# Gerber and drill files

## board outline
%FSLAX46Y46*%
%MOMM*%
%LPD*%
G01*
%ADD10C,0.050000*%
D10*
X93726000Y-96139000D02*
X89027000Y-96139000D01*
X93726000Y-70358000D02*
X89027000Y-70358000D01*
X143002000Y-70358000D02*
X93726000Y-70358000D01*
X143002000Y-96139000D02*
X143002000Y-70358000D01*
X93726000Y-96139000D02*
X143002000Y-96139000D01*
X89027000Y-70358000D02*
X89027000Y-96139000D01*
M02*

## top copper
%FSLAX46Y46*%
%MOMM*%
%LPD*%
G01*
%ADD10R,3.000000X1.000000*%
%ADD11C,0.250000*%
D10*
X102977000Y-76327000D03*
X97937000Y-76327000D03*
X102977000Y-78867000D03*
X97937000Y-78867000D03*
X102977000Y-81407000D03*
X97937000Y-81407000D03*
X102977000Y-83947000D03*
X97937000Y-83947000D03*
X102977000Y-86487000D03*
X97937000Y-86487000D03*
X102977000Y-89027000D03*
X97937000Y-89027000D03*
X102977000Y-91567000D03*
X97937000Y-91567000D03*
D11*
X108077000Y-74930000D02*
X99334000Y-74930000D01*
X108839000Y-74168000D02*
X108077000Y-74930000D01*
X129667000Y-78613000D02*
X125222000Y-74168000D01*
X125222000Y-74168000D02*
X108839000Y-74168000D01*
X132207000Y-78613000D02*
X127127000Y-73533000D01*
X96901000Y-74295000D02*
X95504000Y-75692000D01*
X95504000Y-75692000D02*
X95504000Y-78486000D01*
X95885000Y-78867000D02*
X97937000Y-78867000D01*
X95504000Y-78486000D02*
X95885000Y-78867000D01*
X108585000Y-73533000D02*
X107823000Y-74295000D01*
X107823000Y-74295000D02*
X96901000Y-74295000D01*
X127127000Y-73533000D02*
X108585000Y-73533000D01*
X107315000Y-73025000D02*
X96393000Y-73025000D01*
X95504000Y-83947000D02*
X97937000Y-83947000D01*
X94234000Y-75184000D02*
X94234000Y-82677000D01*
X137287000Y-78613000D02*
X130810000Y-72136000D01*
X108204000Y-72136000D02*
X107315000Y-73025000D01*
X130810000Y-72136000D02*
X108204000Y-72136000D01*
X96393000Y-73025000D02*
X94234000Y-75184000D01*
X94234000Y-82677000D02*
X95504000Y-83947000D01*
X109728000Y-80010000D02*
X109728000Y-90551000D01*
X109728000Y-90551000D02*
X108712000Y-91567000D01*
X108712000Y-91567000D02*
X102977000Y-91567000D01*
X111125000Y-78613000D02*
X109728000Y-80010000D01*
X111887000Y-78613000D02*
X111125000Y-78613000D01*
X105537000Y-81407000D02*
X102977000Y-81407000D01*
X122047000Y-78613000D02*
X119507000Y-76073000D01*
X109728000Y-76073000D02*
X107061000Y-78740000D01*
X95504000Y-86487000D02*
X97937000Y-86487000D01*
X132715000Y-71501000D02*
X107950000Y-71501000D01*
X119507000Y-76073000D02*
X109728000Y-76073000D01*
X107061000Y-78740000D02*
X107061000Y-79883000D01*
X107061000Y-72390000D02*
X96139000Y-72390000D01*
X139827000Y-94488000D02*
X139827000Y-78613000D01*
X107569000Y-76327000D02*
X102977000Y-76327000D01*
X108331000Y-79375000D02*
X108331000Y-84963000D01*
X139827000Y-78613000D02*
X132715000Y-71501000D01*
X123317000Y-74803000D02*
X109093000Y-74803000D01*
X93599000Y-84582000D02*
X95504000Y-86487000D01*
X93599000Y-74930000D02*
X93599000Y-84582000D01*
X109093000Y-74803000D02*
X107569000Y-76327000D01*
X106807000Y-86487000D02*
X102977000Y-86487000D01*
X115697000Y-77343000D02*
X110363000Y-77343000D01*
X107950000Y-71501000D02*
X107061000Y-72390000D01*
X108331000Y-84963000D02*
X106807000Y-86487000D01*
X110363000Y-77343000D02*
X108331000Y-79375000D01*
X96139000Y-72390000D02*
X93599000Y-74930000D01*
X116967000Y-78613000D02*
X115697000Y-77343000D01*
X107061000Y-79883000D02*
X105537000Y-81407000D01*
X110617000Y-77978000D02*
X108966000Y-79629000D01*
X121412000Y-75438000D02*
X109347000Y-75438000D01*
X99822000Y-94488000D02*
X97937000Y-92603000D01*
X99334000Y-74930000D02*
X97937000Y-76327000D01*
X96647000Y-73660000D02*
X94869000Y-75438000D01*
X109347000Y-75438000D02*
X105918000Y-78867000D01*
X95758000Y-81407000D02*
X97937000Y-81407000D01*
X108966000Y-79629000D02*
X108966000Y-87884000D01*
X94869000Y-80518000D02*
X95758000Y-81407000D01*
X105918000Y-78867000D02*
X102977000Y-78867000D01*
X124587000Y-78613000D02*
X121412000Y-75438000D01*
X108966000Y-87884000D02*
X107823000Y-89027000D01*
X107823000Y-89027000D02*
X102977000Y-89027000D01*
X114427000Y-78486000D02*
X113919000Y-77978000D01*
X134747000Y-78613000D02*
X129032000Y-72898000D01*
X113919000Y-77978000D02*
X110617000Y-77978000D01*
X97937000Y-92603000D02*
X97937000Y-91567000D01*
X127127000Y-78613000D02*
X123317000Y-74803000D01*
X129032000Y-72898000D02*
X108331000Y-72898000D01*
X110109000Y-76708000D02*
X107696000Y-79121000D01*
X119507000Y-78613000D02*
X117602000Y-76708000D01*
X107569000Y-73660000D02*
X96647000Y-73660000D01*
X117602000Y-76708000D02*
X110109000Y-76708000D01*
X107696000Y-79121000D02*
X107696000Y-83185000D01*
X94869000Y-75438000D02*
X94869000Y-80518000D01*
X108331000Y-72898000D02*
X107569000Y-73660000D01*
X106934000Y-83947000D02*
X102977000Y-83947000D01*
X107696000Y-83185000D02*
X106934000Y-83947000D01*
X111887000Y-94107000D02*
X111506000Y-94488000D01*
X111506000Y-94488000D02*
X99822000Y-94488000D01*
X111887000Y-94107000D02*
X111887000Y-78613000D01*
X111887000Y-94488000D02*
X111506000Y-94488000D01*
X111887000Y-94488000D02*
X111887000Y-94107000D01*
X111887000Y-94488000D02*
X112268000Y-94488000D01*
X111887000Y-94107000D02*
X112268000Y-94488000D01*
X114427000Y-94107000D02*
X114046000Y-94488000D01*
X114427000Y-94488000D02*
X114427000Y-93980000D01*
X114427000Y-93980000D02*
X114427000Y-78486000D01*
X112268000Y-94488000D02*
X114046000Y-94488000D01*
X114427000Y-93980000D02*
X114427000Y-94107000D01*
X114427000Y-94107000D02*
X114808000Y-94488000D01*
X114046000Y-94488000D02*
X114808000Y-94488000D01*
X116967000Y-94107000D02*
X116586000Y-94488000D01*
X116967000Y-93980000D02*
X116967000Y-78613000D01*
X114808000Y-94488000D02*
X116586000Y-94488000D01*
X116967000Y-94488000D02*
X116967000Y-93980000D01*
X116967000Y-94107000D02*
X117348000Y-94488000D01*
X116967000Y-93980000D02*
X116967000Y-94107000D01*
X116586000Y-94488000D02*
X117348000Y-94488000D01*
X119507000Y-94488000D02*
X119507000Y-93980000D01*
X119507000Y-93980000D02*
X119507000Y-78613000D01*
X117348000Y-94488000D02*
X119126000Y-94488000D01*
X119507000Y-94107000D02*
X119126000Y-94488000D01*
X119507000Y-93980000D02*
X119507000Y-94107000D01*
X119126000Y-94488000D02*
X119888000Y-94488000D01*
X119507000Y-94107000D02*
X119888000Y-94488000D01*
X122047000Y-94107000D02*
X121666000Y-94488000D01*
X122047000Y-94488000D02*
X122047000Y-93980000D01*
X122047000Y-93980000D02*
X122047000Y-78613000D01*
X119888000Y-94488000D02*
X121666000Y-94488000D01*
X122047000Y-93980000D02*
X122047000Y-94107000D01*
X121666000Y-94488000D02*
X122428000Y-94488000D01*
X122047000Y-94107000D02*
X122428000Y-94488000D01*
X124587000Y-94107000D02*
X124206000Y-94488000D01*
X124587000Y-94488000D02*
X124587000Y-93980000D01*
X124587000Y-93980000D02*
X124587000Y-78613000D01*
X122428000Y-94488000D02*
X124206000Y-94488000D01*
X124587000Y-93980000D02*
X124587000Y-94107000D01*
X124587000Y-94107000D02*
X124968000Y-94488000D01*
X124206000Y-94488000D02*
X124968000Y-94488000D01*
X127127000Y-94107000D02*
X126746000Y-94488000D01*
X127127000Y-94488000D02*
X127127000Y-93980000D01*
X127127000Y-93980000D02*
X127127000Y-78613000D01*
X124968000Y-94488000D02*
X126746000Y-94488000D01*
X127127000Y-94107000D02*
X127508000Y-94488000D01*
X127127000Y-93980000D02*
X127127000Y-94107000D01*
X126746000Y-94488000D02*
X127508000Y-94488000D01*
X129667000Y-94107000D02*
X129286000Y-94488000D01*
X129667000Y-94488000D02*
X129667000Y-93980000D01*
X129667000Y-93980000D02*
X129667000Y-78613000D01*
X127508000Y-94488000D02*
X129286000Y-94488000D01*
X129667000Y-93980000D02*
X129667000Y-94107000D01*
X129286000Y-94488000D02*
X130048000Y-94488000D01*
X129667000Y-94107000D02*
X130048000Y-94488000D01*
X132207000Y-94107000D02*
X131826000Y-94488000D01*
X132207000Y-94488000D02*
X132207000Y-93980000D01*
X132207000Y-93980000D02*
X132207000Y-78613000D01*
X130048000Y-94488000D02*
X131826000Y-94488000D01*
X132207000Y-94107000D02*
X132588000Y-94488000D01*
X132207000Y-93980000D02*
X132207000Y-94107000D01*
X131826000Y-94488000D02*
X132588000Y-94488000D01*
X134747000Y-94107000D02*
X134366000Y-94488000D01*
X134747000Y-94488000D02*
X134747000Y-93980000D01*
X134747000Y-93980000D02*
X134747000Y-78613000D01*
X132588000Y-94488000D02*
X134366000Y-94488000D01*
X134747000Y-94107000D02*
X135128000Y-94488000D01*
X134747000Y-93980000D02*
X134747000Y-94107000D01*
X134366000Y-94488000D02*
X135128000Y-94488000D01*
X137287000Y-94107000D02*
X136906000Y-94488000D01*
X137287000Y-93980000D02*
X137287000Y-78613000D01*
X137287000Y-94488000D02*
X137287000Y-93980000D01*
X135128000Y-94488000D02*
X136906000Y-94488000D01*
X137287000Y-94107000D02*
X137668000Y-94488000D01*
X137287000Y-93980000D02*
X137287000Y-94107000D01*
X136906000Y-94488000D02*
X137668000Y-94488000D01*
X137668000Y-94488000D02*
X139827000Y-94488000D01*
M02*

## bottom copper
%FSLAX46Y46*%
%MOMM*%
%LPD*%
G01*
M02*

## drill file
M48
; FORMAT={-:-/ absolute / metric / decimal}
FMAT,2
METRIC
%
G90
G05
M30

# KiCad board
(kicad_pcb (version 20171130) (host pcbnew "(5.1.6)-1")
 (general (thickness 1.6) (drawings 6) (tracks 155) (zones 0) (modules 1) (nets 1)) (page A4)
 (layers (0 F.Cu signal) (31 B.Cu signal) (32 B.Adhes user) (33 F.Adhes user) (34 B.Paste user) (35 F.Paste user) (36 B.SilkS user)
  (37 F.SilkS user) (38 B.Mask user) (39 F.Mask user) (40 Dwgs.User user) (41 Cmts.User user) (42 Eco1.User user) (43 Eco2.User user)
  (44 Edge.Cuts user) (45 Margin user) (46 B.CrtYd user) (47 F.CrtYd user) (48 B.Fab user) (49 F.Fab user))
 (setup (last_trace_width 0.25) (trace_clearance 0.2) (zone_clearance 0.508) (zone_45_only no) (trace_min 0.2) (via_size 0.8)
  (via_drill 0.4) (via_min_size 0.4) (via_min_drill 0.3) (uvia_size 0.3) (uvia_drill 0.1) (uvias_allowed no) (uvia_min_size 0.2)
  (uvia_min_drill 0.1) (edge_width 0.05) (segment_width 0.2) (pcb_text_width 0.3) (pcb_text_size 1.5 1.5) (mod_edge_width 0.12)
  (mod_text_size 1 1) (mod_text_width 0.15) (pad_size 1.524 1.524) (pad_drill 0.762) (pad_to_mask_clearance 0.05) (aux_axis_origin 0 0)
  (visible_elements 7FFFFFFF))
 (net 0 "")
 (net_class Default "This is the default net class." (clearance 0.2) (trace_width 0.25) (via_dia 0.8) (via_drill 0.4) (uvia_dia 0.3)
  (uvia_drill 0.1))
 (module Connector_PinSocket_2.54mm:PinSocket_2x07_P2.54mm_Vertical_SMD (layer F.Cu) (at 100.457 83.947)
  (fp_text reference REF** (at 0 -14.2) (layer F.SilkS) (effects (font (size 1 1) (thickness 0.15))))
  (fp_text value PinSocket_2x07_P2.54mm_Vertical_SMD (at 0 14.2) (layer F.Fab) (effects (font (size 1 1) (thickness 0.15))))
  (pad 1 smd rect (at 2.52 -7.62) (size 3 1) (layers F.Cu F.Paste F.Mask))
  (pad 2 smd rect (at -2.52 -7.62) (size 3 1) (layers F.Cu F.Paste F.Mask))
  (pad 3 smd rect (at 2.52 -5.08) (size 3 1) (layers F.Cu F.Paste F.Mask))
  (pad 4 smd rect (at -2.52 -5.08) (size 3 1) (layers F.Cu F.Paste F.Mask))
  (pad 5 smd rect (at 2.52 -2.54) (size 3 1) (layers F.Cu F.Paste F.Mask))
  (pad 6 smd rect (at -2.52 -2.54) (size 3 1) (layers F.Cu F.Paste F.Mask))
  (pad 7 smd rect (at 2.52 0) (size 3 1) (layers F.Cu F.Paste F.Mask))
  (pad 8 smd rect (at -2.52 0) (size 3 1) (layers F.Cu F.Paste F.Mask))
  (pad 9 smd rect (at 2.52 2.54) (size 3 1) (layers F.Cu F.Paste F.Mask))
  (pad 10 smd rect (at -2.52 2.54) (size 3 1) (layers F.Cu F.Paste F.Mask))
  (pad 11 smd rect (at 2.52 5.08) (size 3 1) (layers F.Cu F.Paste F.Mask))
  (pad 12 smd rect (at -2.52 5.08) (size 3 1) (layers F.Cu F.Paste F.Mask))
  (pad 13 smd rect (at 2.52 7.62) (size 3 1) (layers F.Cu F.Paste F.Mask))
  (pad 14 smd rect (at -2.52 7.62) (size 3 1) (layers F.Cu F.Paste F.Mask)))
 (gr_line (start 93.726 96.139) (end 89.027 96.139) (layer Edge.Cuts) (width 0.05))
 (gr_line (start 93.726 70.358) (end 89.027 70.358) (layer Edge.Cuts) (width 0.05))
 (gr_line (start 143.002 70.358) (end 93.726 70.358) (layer Edge.Cuts) (width 0.05))
 (gr_line (start 143.002 96.139) (end 143.002 70.358) (layer Edge.Cuts) (width 0.05))
 (gr_line (start 93.726 96.139) (end 143.002 96.139) (layer Edge.Cuts) (width 0.05))
 (gr_line (start 89.027 70.358) (end 89.027 96.139) (layer Edge.Cuts) (width 0.05))
 (segment (start 108.077 74.93) (end 99.334 74.93) (width 0.25) (layer F.Cu) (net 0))
 (segment (start 108.839 74.168) (end 108.077 74.93) (width 0.25) (layer F.Cu) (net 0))
 (segment (start 129.667 78.613) (end 125.222 74.168) (width 0.25) (layer F.Cu) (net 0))
 (segment (start 125.222 74.168) (end 108.839 74.168) (width 0.25) (layer F.Cu) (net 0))
 (segment (start 132.207 78.613) (end 127.127 73.533) (width 0.25) (layer F.Cu) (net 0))
 (segment (start 96.901 74.295) (end 95.504 75.692) (width 0.25) (layer F.Cu) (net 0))
 (segment (start 95.504 75.692) (end 95.504 78.486) (width 0.25) (layer F.Cu) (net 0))
 (segment (start 95.885 78.867) (end 97.937 78.867) (width 0.25) (layer F.Cu) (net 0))
 (segment (start 95.504 78.486) (end 95.885 78.867) (width 0.25) (layer F.Cu) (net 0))
 (segment (start 108.585 73.533) (end 107.823 74.295) (width 0.25) (layer F.Cu) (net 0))
 (segment (start 107.823 74.295) (end 96.901 74.295) (width 0.25) (layer F.Cu) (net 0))
 (segment (start 127.127 73.533) (end 108.585 73.533) (width 0.25) (layer F.Cu) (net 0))
 (segment (start 107.315 73.025) (end 96.393 73.025) (width 0.25) (layer F.Cu) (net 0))
 (segment (start 95.504 83.947) (end 97.937 83.947) (width 0.25) (layer F.Cu) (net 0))
 (segment (start 94.234 75.184) (end 94.234 82.677) (width 0.25) (layer F.Cu) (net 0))
 (segment (start 137.287 78.613) (end 130.81 72.136) (width 0.25) (layer F.Cu) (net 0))
 (segment (start 108.204 72.136) (end 107.315 73.025) (width 0.25) (layer F.Cu) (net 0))
 (segment (start 130.81 72.136) (end 108.204 72.136) (width 0.25) (layer F.Cu) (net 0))
 (segment (start 96.393 73.025) (end 94.234 75.184) (width 0.25) (layer F.Cu) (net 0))
 (segment (start 94.234 82.677) (end 95.504 83.947) (width 0.25) (layer F.Cu) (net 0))
 (segment (start 109.728 80.01) (end 109.728 90.551) (width 0.25) (layer F.Cu) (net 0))
 (segment (start 109.728 90.551) (end 108.712 91.567) (width 0.25) (layer F.Cu) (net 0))
 (segment (start 108.712 91.567) (end 102.977 91.567) (width 0.25) (layer F.Cu) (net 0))
 (segment (start 111.125 78.613) (end 109.728 80.01) (width 0.25) (layer F.Cu) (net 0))
 (segment (start 111.887 78.613) (end 111.125 78.613) (width 0.25) (layer F.Cu) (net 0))
 (segment (start 105.537 81.407) (end 102.977 81.407) (width 0.25) (layer F.Cu) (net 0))
 (segment (start 122.047 78.613) (end 119.507 76.073) (width 0.25) (layer F.Cu) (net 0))
 (segment (start 109.728 76.073) (end 107.061 78.74) (width 0.25) (layer F.Cu) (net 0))
 (segment (start 95.504 86.487) (end 97.937 86.487) (width 0.25) (layer F.Cu) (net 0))
 (segment (start 132.715 71.501) (end 107.95 71.501) (width 0.25) (layer F.Cu) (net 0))
 (segment (start 119.507 76.073) (end 109.728 76.073) (width 0.25) (layer F.Cu) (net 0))
 (segment (start 107.061 78.74) (end 107.061 79.883) (width 0.25) (layer F.Cu) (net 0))
 (segment (start 107.061 72.39) (end 96.139 72.39) (width 0.25) (layer F.Cu) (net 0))
 (segment (start 139.827 94.488) (end 139.827 78.613) (width 0.25) (layer F.Cu) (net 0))
 (segment (start 107.569 76.327) (end 102.977 76.327) (width 0.25) (layer F.Cu) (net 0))
 (segment (start 108.331 79.375) (end 108.331 84.963) (width 0.25) (layer F.Cu) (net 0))
 (segment (start 139.827 78.613) (end 132.715 71.501) (width 0.25) (layer F.Cu) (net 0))
 (segment (start 123.317 74.803) (end 109.093 74.803) (width 0.25) (layer F.Cu) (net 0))
 (segment (start 93.599 84.582) (end 95.504 86.487) (width 0.25) (layer F.Cu) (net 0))
 (segment (start 93.599 74.93) (end 93.599 84.582) (width 0.25) (layer F.Cu) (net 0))
 (segment (start 109.093 74.803) (end 107.569 76.327) (width 0.25) (layer F.Cu) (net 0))
 (segment (start 106.807 86.487) (end 102.977 86.487) (width 0.25) (layer F.Cu) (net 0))
 (segment (start 115.697 77.343) (end 110.363 77.343) (width 0.25) (layer F.Cu) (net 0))
 (segment (start 107.95 71.501) (end 107.061 72.39) (width 0.25) (layer F.Cu) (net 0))
 (segment (start 108.331 84.963) (end 106.807 86.487) (width 0.25) (layer F.Cu) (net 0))
 (segment (start 110.363 77.343) (end 108.331 79.375) (width 0.25) (layer F.Cu) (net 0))
 (segment (start 96.139 72.39) (end 93.599 74.93) (width 0.25) (layer F.Cu) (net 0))
 (segment (start 116.967 78.613) (end 115.697 77.343) (width 0.25) (layer F.Cu) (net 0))
 (segment (start 107.061 79.883) (end 105.537 81.407) (width 0.25) (layer F.Cu) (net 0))
 (segment (start 110.617 77.978) (end 108.966 79.629) (width 0.25) (layer F.Cu) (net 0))
 (segment (start 121.412 75.438) (end 109.347 75.438) (width 0.25) (layer F.Cu) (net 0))
 (segment (start 99.822 94.488) (end 97.937 92.603) (width 0.25) (layer F.Cu) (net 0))
 (segment (start 99.334 74.93) (end 97.937 76.327) (width 0.25) (layer F.Cu) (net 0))
 (segment (start 96.647 73.66) (end 94.869 75.438) (width 0.25) (layer F.Cu) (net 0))
 (segment (start 109.347 75.438) (end 105.918 78.867) (width 0.25) (layer F.Cu) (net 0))
 (segment (start 95.758 81.407) (end 97.937 81.407) (width 0.25) (layer F.Cu) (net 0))
 (segment (start 108.966 79.629) (end 108.966 87.884) (width 0.25) (layer F.Cu) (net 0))
 (segment (start 94.869 80.518) (end 95.758 81.407) (width 0.25) (layer F.Cu) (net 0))
 (segment (start 105.918 78.867) (end 102.977 78.867) (width 0.25) (layer F.Cu) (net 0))
 (segment (start 124.587 78.613) (end 121.412 75.438) (width 0.25) (layer F.Cu) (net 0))
 (segment (start 108.966 87.884) (end 107.823 89.027) (width 0.25) (layer F.Cu) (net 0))
 (segment (start 107.823 89.027) (end 102.977 89.027) (width 0.25) (layer F.Cu) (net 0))
 (segment (start 114.427 78.486) (end 113.919 77.978) (width 0.25) (layer F.Cu) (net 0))
 (segment (start 134.747 78.613) (end 129.032 72.898) (width 0.25) (layer F.Cu) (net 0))
 (segment (start 113.919 77.978) (end 110.617 77.978) (width 0.25) (layer F.Cu) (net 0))
 (segment (start 97.937 92.603) (end 97.937 91.567) (width 0.25) (layer F.Cu) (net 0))
 (segment (start 127.127 78.613) (end 123.317 74.803) (width 0.25) (layer F.Cu) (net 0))
 (segment (start 129.032 72.898) (end 108.331 72.898) (width 0.25) (layer F.Cu) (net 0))
 (segment (start 110.109 76.708) (end 107.696 79.121) (width 0.25) (layer F.Cu) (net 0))
 (segment (start 119.507 78.613) (end 117.602 76.708) (width 0.25) (layer F.Cu) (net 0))
 (segment (start 107.569 73.66) (end 96.647 73.66) (width 0.25) (layer F.Cu) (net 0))
 (segment (start 117.602 76.708) (end 110.109 76.708) (width 0.25) (layer F.Cu) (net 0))
 (segment (start 107.696 79.121) (end 107.696 83.185) (width 0.25) (layer F.Cu) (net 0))
 (segment (start 94.869 75.438) (end 94.869 80.518) (width 0.25) (layer F.Cu) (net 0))
 (segment (start 108.331 72.898) (end 107.569 73.66) (width 0.25) (layer F.Cu) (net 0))
 (segment (start 106.934 83.947) (end 102.977 83.947) (width 0.25) (layer F.Cu) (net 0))
 (segment (start 107.696 83.185) (end 106.934 83.947) (width 0.25) (layer F.Cu) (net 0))
 (segment (start 111.887 94.107) (end 111.506 94.488) (width 0.25) (layer F.Cu) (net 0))
 (segment (start 111.506 94.488) (end 99.822 94.488) (width 0.25) (layer F.Cu) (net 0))
 (segment (start 111.887 94.107) (end 111.887 78.613) (width 0.25) (layer F.Cu) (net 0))
 (segment (start 111.887 94.488) (end 111.506 94.488) (width 0.25) (layer F.Cu) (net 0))
 (segment (start 111.887 94.488) (end 111.887 94.107) (width 0.25) (layer F.Cu) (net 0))
 (segment (start 111.887 94.488) (end 112.268 94.488) (width 0.25) (layer F.Cu) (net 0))
 (segment (start 111.887 94.107) (end 112.268 94.488) (width 0.25) (layer F.Cu) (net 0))
 (segment (start 114.427 94.107) (end 114.046 94.488) (width 0.25) (layer F.Cu) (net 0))
 (segment (start 114.427 94.488) (end 114.427 93.98) (width 0.25) (layer F.Cu) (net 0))
 (segment (start 114.427 93.98) (end 114.427 78.486) (width 0.25) (layer F.Cu) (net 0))
 (segment (start 112.268 94.488) (end 114.046 94.488) (width 0.25) (layer F.Cu) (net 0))
 (segment (start 114.427 93.98) (end 114.427 94.107) (width 0.25) (layer F.Cu) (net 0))
 (segment (start 114.427 94.107) (end 114.808 94.488) (width 0.25) (layer F.Cu) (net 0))
 (segment (start 114.046 94.488) (end 114.808 94.488) (width 0.25) (layer F.Cu) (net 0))
 (segment (start 116.967 94.107) (end 116.586 94.488) (width 0.25) (layer F.Cu) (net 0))
 (segment (start 116.967 93.98) (end 116.967 78.613) (width 0.25) (layer F.Cu) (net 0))
 (segment (start 114.808 94.488) (end 116.586 94.488) (width 0.25) (layer F.Cu) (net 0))
 (segment (start 116.967 94.488) (end 116.967 93.98) (width 0.25) (layer F.Cu) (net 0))
 (segment (start 116.967 94.107) (end 117.348 94.488) (width 0.25) (layer F.Cu) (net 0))
 (segment (start 116.967 93.98) (end 116.967 94.107) (width 0.25) (layer F.Cu) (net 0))
 (segment (start 116.586 94.488) (end 117.348 94.488) (width 0.25) (layer F.Cu) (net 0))
 (segment (start 119.507 94.488) (end 119.507 93.98) (width 0.25) (layer F.Cu) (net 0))
 (segment (start 119.507 93.98) (end 119.507 78.613) (width 0.25) (layer F.Cu) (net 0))
 (segment (start 117.348 94.488) (end 119.126 94.488) (width 0.25) (layer F.Cu) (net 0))
 (segment (start 119.507 94.107) (end 119.126 94.488) (width 0.25) (layer F.Cu) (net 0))
 (segment (start 119.507 93.98) (end 119.507 94.107) (width 0.25) (layer F.Cu) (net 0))
 (segment (start 119.126 94.488) (end 119.888 94.488) (width 0.25) (layer F.Cu) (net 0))
 (segment (start 119.507 94.107) (end 119.888 94.488) (width 0.25) (layer F.Cu) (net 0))
 (segment (start 122.047 94.107) (end 121.666 94.488) (width 0.25) (layer F.Cu) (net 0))
 (segment (start 122.047 94.488) (end 122.047 93.98) (width 0.25) (layer F.Cu) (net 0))
 (segment (start 122.047 93.98) (end 122.047 78.613) (width 0.25) (layer F.Cu) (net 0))
 (segment (start 119.888 94.488) (end 121.666 94.488) (width 0.25) (layer F.Cu) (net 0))
 (segment (start 122.047 93.98) (end 122.047 94.107) (width 0.25) (layer F.Cu) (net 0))
 (segment (start 121.666 94.488) (end 122.428 94.488) (width 0.25) (layer F.Cu) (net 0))
 (segment (start 122.047 94.107) (end 122.428 94.488) (width 0.25) (layer F.Cu) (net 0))
 (segment (start 124.587 94.107) (end 124.206 94.488) (width 0.25) (layer F.Cu) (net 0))
 (segment (start 124.587 94.488) (end 124.587 93.98) (width 0.25) (layer F.Cu) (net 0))
 (segment (start 124.587 93.98) (end 124.587 78.613) (width 0.25) (layer F.Cu) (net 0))
 (segment (start 122.428 94.488) (end 124.206 94.488) (width 0.25) (layer F.Cu) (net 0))
 (segment (start 124.587 93.98) (end 124.587 94.107) (width 0.25) (layer F.Cu) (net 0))
 (segment (start 124.587 94.107) (end 124.968 94.488) (width 0.25) (layer F.Cu) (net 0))
 (segment (start 124.206 94.488) (end 124.968 94.488) (width 0.25) (layer F.Cu) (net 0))
 (segment (start 127.127 94.107) (end 126.746 94.488) (width 0.25) (layer F.Cu) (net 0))
 (segment (start 127.127 94.488) (end 127.127 93.98) (width 0.25) (layer F.Cu) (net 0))
 (segment (start 127.127 93.98) (end 127.127 78.613) (width 0.25) (layer F.Cu) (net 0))
 (segment (start 124.968 94.488) (end 126.746 94.488) (width 0.25) (layer F.Cu) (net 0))
 (segment (start 127.127 94.107) (end 127.508 94.488) (width 0.25) (layer F.Cu) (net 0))
 (segment (start 127.127 93.98) (end 127.127 94.107) (width 0.25) (layer F.Cu) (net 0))
 (segment (start 126.746 94.488) (end 127.508 94.488) (width 0.25) (layer F.Cu) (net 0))
 (segment (start 129.667 94.107) (end 129.286 94.488) (width 0.25) (layer F.Cu) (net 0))
 (segment (start 129.667 94.488) (end 129.667 93.98) (width 0.25) (layer F.Cu) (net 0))
 (segment (start 129.667 93.98) (end 129.667 78.613) (width 0.25) (layer F.Cu) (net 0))
 (segment (start 127.508 94.488) (end 129.286 94.488) (width 0.25) (layer F.Cu) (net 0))
 (segment (start 129.667 93.98) (end 129.667 94.107) (width 0.25) (layer F.Cu) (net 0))
 (segment (start 129.286 94.488) (end 130.048 94.488) (width 0.25) (layer F.Cu) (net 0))
 (segment (start 129.667 94.107) (end 130.048 94.488) (width 0.25) (layer F.Cu) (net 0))
 (segment (start 132.207 94.107) (end 131.826 94.488) (width 0.25) (layer F.Cu) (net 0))
 (segment (start 132.207 94.488) (end 132.207 93.98) (width 0.25) (layer F.Cu) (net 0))
 (segment (start 132.207 93.98) (end 132.207 78.613) (width 0.25) (layer F.Cu) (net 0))
 (segment (start 130.048 94.488) (end 131.826 94.488) (width 0.25) (layer F.Cu) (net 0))
 (segment (start 132.207 94.107) (end 132.588 94.488) (width 0.25) (layer F.Cu) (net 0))
 (segment (start 132.207 93.98) (end 132.207 94.107) (width 0.25) (layer F.Cu) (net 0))
 (segment (start 131.826 94.488) (end 132.588 94.488) (width 0.25) (layer F.Cu) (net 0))
 (segment (start 134.747 94.107) (end 134.366 94.488) (width 0.25) (layer F.Cu) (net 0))
 (segment (start 134.747 94.488) (end 134.747 93.98) (width 0.25) (layer F.Cu) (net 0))
 (segment (start 134.747 93.98) (end 134.747 78.613) (width 0.25) (layer F.Cu) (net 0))
 (segment (start 132.588 94.488) (end 134.366 94.488) (width 0.25) (layer F.Cu) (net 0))
 (segment (start 134.747 94.107) (end 135.128 94.488) (width 0.25) (layer F.Cu) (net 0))
 (segment (start 134.747 93.98) (end 134.747 94.107) (width 0.25) (layer F.Cu) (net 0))
 (segment (start 134.366 94.488) (end 135.128 94.488) (width 0.25) (layer F.Cu) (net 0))
 (segment (start 137.287 94.107) (end 136.906 94.488) (width 0.25) (layer F.Cu) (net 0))
 (segment (start 137.287 93.98) (end 137.287 78.613) (width 0.25) (layer F.Cu) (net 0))
 (segment (start 137.287 94.488) (end 137.287 93.98) (width 0.25) (layer F.Cu) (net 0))
 (segment (start 135.128 94.488) (end 136.906 94.488) (width 0.25) (layer F.Cu) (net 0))
 (segment (start 137.287 94.107) (end 137.668 94.488) (width 0.25) (layer F.Cu) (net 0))
 (segment (start 137.287 93.98) (end 137.287 94.107) (width 0.25) (layer F.Cu) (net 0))
 (segment (start 136.906 94.488) (end 137.668 94.488) (width 0.25) (layer F.Cu) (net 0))
 (segment (start 137.668 94.488) (end 139.827 94.488) (width 0.25) (layer F.Cu) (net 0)))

